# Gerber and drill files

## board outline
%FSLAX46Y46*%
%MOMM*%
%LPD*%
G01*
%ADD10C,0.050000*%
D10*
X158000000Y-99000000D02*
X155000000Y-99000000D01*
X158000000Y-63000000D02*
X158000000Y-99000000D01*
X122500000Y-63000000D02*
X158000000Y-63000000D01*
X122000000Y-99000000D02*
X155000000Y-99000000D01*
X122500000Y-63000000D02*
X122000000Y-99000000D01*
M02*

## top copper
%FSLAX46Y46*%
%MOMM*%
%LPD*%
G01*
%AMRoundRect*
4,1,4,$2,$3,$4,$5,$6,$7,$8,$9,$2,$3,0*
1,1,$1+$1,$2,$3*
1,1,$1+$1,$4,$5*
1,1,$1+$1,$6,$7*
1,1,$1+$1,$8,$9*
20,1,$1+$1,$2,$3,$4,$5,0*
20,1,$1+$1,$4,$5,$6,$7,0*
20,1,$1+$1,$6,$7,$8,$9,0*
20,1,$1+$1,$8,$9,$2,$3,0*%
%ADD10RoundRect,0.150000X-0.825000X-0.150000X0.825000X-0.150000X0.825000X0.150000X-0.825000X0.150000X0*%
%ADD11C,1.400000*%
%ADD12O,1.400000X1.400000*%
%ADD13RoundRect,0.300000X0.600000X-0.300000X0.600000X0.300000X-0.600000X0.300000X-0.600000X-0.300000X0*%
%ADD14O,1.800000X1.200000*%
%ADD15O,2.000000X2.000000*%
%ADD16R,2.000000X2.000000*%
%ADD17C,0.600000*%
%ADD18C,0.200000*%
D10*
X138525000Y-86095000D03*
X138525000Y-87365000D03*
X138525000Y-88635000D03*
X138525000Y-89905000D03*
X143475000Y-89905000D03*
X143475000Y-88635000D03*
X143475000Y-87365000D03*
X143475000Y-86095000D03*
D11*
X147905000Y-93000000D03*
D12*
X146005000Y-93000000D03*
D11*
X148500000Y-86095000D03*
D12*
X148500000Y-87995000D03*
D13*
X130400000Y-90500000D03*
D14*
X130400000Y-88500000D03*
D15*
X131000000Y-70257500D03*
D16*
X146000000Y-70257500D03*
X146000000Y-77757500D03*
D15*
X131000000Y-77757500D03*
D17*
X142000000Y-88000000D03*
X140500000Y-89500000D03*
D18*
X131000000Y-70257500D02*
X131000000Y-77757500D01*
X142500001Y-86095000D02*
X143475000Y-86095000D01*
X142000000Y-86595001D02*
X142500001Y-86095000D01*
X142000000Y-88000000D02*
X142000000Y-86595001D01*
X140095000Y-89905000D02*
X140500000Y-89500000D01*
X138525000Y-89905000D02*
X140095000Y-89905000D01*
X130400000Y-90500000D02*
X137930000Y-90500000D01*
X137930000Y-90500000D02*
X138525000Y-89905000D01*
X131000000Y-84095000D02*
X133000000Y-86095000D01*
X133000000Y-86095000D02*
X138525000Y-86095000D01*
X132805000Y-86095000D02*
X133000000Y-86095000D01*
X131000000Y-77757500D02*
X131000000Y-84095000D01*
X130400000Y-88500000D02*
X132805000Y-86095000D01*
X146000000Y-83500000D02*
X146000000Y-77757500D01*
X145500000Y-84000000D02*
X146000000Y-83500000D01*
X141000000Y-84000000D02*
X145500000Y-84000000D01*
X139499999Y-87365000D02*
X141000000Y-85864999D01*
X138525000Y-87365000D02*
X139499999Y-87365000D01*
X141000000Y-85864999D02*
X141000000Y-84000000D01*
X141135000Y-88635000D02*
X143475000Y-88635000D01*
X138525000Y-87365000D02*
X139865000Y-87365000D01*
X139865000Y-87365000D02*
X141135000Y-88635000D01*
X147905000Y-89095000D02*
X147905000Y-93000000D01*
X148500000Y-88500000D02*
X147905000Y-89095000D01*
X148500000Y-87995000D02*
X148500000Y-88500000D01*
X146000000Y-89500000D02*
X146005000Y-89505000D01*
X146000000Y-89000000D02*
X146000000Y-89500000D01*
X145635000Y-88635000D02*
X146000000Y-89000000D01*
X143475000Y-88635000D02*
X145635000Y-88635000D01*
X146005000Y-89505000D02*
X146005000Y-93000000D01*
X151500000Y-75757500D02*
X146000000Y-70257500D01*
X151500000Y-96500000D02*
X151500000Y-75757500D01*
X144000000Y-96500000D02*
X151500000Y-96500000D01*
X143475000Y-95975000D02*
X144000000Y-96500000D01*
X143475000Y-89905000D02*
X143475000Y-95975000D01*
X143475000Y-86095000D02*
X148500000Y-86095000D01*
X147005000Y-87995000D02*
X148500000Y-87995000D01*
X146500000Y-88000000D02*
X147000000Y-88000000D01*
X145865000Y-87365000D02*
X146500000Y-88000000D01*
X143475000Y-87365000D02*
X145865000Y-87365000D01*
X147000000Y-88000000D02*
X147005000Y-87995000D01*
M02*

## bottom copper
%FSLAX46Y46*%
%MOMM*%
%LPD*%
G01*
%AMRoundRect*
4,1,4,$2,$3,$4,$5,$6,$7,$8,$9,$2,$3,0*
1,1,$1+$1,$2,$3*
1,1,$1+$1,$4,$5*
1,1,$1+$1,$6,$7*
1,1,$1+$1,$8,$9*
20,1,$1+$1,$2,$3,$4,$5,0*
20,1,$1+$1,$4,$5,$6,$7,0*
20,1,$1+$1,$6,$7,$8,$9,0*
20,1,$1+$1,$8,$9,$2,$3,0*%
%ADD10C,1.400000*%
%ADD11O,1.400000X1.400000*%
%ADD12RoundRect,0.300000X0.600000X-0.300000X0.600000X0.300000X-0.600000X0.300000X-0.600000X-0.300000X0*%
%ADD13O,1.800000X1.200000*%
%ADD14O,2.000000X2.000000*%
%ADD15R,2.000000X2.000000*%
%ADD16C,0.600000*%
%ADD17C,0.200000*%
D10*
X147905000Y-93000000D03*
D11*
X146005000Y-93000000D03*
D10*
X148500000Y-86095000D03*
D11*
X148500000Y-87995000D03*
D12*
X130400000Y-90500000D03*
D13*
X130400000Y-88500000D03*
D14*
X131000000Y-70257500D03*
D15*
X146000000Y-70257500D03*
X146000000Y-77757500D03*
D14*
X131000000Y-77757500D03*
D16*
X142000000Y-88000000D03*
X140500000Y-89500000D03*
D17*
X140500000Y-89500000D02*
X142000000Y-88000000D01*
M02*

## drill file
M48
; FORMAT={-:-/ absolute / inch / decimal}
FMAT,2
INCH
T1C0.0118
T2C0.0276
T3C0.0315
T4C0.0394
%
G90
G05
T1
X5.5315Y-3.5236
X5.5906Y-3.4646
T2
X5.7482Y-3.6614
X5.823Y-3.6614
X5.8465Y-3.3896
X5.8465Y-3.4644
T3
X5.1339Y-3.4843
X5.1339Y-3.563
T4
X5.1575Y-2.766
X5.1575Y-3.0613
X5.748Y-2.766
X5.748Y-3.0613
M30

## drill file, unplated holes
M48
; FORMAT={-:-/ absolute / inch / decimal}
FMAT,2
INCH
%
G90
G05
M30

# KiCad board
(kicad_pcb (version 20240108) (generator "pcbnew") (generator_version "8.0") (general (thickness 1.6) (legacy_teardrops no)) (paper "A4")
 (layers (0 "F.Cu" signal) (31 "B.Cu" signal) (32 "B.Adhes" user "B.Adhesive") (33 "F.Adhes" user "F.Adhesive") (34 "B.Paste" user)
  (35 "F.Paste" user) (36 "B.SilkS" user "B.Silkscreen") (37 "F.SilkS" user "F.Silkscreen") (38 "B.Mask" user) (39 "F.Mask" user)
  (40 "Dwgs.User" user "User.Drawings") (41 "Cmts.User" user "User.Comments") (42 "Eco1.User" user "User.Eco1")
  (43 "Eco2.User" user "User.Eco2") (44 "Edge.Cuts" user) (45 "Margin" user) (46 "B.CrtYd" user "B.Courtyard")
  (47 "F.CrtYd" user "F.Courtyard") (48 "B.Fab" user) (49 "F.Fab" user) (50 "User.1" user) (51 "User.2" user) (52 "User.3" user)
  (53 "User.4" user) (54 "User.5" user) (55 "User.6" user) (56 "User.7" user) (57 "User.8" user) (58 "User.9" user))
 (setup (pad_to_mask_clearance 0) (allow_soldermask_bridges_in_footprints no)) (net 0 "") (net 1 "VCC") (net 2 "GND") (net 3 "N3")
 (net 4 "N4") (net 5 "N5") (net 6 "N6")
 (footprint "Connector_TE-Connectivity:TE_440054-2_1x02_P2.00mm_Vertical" (layer "F.Cu") (at 130.4 90.5 90)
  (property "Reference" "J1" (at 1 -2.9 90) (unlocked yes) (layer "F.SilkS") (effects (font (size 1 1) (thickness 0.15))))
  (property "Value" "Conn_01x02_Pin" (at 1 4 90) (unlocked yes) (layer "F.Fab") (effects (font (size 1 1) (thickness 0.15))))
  (pad "1" thru_hole roundrect (at 0 0 90) (size 1.2 1.8) (drill 0.8) (layers "*.Cu" "*.Mask") (remove_unused_layers no)
   (roundrect_rratio 0.25) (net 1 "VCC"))
  (pad "2" thru_hole oval (at 2 0 90) (size 1.2 1.8) (drill 0.8) (layers "*.Cu" "*.Mask") (remove_unused_layers no) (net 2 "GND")))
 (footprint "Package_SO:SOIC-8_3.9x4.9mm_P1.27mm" (layer "F.Cu") (at 141 88)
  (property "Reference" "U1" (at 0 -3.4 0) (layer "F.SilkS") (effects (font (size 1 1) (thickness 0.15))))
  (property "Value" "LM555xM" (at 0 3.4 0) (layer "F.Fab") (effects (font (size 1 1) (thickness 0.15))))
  (pad "1" smd roundrect (at -2.475 -1.905) (size 1.95 0.6) (layers "F.Cu" "F.Paste" "F.Mask") (roundrect_rratio 0.25) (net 2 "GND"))
  (pad "2" smd roundrect (at -2.475 -0.635) (size 1.95 0.6) (layers "F.Cu" "F.Paste" "F.Mask") (roundrect_rratio 0.25) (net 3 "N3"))
  (pad "3" smd roundrect (at -2.475 0.635) (size 1.95 0.6) (layers "F.Cu" "F.Paste" "F.Mask") (roundrect_rratio 0.25) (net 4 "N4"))
  (pad "4" smd roundrect (at -2.475 1.905) (size 1.95 0.6) (layers "F.Cu" "F.Paste" "F.Mask") (roundrect_rratio 0.25) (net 1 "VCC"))
  (pad "5" smd roundrect (at 2.475 1.905) (size 1.95 0.6) (layers "F.Cu" "F.Paste" "F.Mask") (roundrect_rratio 0.25) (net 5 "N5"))
  (pad "6" smd roundrect (at 2.475 0.635) (size 1.95 0.6) (layers "F.Cu" "F.Paste" "F.Mask") (roundrect_rratio 0.25) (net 3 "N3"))
  (pad "7" smd roundrect (at 2.475 -0.635) (size 1.95 0.6) (layers "F.Cu" "F.Paste" "F.Mask") (roundrect_rratio 0.25) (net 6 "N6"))
  (pad "8" smd roundrect (at 2.475 -1.905) (size 1.95 0.6) (layers "F.Cu" "F.Paste" "F.Mask") (roundrect_rratio 0.25) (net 1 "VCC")))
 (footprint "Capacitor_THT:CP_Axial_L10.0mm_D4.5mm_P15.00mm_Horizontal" (layer "F.Cu") (at 146 77.7575 180)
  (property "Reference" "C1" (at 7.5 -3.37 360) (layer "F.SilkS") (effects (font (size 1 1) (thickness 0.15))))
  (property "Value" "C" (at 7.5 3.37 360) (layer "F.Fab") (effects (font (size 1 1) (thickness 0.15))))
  (pad "1" thru_hole rect (at 0 0 180) (size 2 2) (drill 1) (layers "*.Cu" "*.Mask") (remove_unused_layers no) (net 3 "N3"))
  (pad "2" thru_hole oval (at 15 0 180) (size 2 2) (drill 1) (layers "*.Cu" "*.Mask") (remove_unused_layers no) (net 2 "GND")))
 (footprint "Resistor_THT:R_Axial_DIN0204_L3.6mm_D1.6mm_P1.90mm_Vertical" (layer "F.Cu") (at 147.905 93 180)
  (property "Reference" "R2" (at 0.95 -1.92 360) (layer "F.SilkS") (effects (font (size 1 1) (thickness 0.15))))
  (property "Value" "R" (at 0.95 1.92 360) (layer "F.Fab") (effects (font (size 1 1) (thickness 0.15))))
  (pad "1" thru_hole circle (at 0 0 180) (size 1.4 1.4) (drill 0.7) (layers "*.Cu" "*.Mask") (remove_unused_layers no) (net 6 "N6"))
  (pad "2" thru_hole oval (at 1.9 0 180) (size 1.4 1.4) (drill 0.7) (layers "*.Cu" "*.Mask") (remove_unused_layers no) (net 3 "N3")))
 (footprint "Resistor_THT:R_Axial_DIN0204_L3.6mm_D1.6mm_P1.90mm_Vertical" (layer "F.Cu") (at 148.5 86.095 -90)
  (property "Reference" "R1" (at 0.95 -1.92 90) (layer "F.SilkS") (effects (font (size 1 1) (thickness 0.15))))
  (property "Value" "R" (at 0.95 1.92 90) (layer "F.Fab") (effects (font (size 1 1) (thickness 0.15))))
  (pad "1" thru_hole circle (at 0 0 270) (size 1.4 1.4) (drill 0.7) (layers "*.Cu" "*.Mask") (remove_unused_layers no) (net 1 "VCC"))
  (pad "2" thru_hole oval (at 1.9 0 270) (size 1.4 1.4) (drill 0.7) (layers "*.Cu" "*.Mask") (remove_unused_layers no) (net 6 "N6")))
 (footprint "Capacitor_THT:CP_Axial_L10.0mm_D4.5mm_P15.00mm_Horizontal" (layer "F.Cu") (at 146 70.2575 180)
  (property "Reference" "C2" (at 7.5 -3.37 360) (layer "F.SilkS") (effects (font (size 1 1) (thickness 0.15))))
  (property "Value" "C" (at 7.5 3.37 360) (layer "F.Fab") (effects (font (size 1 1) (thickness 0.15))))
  (pad "1" thru_hole rect (at 0 0 180) (size 2 2) (drill 1) (layers "*.Cu" "*.Mask") (remove_unused_layers no) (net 5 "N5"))
  (pad "2" thru_hole oval (at 15 0 180) (size 2 2) (drill 1) (layers "*.Cu" "*.Mask") (remove_unused_layers no) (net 2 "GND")))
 (gr_line (start 122 99) (end 155 99) (stroke (width 0.05) (type default)) (layer "Edge.Cuts"))
 (gr_line (start 122.5 63) (end 122 99) (stroke (width 0.05) (type default)) (layer "Edge.Cuts"))
 (gr_line (start 158 99) (end 155 99) (stroke (width 0.05) (type default)) (layer "Edge.Cuts"))
 (gr_line (start 158 63) (end 158 99) (stroke (width 0.05) (type default)) (layer "Edge.Cuts"))
 (gr_line (start 122.5 63) (end 158 63) (stroke (width 0.05) (type default)) (layer "Edge.Cuts"))
 (segment (start 131 84.095) (end 133 86.095) (width 0.2) (layer "F.Cu") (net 2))
 (segment (start 133 86.095) (end 138.525 86.095) (width 0.2) (layer "F.Cu") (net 2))
 (segment (start 131 77.7575) (end 131 84.095) (width 0.2) (layer "F.Cu") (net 2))
 (segment (start 132.805 86.095) (end 133 86.095) (width 0.2) (layer "F.Cu") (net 2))
 (segment (start 130.4 88.5) (end 132.805 86.095) (width 0.2) (layer "F.Cu") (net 2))
 (segment (start 131 70.2575) (end 131 77.7575) (width 0.2) (layer "F.Cu") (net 2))
 (segment (start 139.865 87.365) (end 141.135 88.635) (width 0.2) (layer "F.Cu") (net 3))
 (segment (start 141 85.864999) (end 141 84) (width 0.2) (layer "F.Cu") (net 3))
 (segment (start 146 89) (end 146 89.5) (width 0.2) (layer "F.Cu") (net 3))
 (segment (start 146 89.5) (end 146.005 89.505) (width 0.2) (layer "F.Cu") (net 3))
 (segment (start 141.135 88.635) (end 143.475 88.635) (width 0.2) (layer "F.Cu") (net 3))
 (segment (start 146.005 89.505) (end 146.005 93) (width 0.2) (layer "F.Cu") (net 3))
 (segment (start 139.499999 87.365) (end 141 85.864999) (width 0.2) (layer "F.Cu") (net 3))
 (segment (start 145.635 88.635) (end 146 89) (width 0.2) (layer "F.Cu") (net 3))
 (segment (start 138.525 87.365) (end 139.865 87.365) (width 0.2) (layer "F.Cu") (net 3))
 (segment (start 146 83.5) (end 146 77.7575) (width 0.2) (layer "F.Cu") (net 3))
 (segment (start 138.525 87.365) (end 139.499999 87.365) (width 0.2) (layer "F.Cu") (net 3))
 (segment (start 143.475 88.635) (end 145.635 88.635) (width 0.2) (layer "F.Cu") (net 3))
 (segment (start 141 84) (end 145.5 84) (width 0.2) (layer "F.Cu") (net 3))
 (segment (start 145.5 84) (end 146 83.5) (width 0.2) (layer "F.Cu") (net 3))
 (segment (start 151.5 96.5) (end 151.5 75.7575) (width 0.2) (layer "F.Cu") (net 5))
 (segment (start 144 96.5) (end 151.5 96.5) (width 0.2) (layer "F.Cu") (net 5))
 (segment (start 151.5 75.7575) (end 146 70.2575) (width 0.2) (layer "F.Cu") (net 5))
 (segment (start 143.475 89.905) (end 143.475 95.975) (width 0.2) (layer "F.Cu") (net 5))
 (segment (start 143.475 95.975) (end 144 96.5) (width 0.2) (layer "F.Cu") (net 5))
 (segment (start 142 88) (end 142 86.595001) (width 0.2) (layer "F.Cu") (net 1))
 (segment (start 137.93 90.5) (end 138.525 89.905) (width 0.2) (layer "F.Cu") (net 1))
 (segment (start 138.525 89.905) (end 140.095 89.905) (width 0.2) (layer "F.Cu") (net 1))
 (segment (start 140.095 89.905) (end 140.5 89.5) (width 0.2) (layer "F.Cu") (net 1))
 (segment (start 142.500001 86.095) (end 143.475 86.095) (width 0.2) (layer "F.Cu") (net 1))
 (segment (start 142 86.595001) (end 142.500001 86.095) (width 0.2) (layer "F.Cu") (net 1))
 (segment (start 143.475 86.095) (end 148.5 86.095) (width 0.2) (layer "F.Cu") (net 1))
 (segment (start 130.4 90.5) (end 137.93 90.5) (width 0.2) (layer "F.Cu") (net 1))
 (via (at 142 88) (size 0.6) (drill 0.3) (layers "F.Cu" "B.Cu") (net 1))
 (via (at 140.5 89.5) (size 0.6) (drill 0.3) (layers "F.Cu" "B.Cu") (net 1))
 (segment (start 140.5 89.5) (end 142 88) (width 0.2) (layer "B.Cu") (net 1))
 (segment (start 147.905 89.095) (end 147.905 93) (width 0.2) (layer "F.Cu") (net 6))
 (segment (start 148.5 87.995) (end 148.5 88.5) (width 0.2) (layer "F.Cu") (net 6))
 (segment (start 148.5 88.5) (end 147.905 89.095) (width 0.2) (layer "F.Cu") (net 6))
 (segment (start 146.5 88) (end 147 88) (width 0.2) (layer "F.Cu") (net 6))
 (segment (start 145.865 87.365) (end 146.5 88) (width 0.2) (layer "F.Cu") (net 6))
 (segment (start 143.475 87.365) (end 145.865 87.365) (width 0.2) (layer "F.Cu") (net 6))
 (segment (start 147.005 87.995) (end 148.5 87.995) (width 0.2) (layer "F.Cu") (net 6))
 (segment (start 147 88) (end 147.005 87.995) (width 0.2) (layer "F.Cu") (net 6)))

